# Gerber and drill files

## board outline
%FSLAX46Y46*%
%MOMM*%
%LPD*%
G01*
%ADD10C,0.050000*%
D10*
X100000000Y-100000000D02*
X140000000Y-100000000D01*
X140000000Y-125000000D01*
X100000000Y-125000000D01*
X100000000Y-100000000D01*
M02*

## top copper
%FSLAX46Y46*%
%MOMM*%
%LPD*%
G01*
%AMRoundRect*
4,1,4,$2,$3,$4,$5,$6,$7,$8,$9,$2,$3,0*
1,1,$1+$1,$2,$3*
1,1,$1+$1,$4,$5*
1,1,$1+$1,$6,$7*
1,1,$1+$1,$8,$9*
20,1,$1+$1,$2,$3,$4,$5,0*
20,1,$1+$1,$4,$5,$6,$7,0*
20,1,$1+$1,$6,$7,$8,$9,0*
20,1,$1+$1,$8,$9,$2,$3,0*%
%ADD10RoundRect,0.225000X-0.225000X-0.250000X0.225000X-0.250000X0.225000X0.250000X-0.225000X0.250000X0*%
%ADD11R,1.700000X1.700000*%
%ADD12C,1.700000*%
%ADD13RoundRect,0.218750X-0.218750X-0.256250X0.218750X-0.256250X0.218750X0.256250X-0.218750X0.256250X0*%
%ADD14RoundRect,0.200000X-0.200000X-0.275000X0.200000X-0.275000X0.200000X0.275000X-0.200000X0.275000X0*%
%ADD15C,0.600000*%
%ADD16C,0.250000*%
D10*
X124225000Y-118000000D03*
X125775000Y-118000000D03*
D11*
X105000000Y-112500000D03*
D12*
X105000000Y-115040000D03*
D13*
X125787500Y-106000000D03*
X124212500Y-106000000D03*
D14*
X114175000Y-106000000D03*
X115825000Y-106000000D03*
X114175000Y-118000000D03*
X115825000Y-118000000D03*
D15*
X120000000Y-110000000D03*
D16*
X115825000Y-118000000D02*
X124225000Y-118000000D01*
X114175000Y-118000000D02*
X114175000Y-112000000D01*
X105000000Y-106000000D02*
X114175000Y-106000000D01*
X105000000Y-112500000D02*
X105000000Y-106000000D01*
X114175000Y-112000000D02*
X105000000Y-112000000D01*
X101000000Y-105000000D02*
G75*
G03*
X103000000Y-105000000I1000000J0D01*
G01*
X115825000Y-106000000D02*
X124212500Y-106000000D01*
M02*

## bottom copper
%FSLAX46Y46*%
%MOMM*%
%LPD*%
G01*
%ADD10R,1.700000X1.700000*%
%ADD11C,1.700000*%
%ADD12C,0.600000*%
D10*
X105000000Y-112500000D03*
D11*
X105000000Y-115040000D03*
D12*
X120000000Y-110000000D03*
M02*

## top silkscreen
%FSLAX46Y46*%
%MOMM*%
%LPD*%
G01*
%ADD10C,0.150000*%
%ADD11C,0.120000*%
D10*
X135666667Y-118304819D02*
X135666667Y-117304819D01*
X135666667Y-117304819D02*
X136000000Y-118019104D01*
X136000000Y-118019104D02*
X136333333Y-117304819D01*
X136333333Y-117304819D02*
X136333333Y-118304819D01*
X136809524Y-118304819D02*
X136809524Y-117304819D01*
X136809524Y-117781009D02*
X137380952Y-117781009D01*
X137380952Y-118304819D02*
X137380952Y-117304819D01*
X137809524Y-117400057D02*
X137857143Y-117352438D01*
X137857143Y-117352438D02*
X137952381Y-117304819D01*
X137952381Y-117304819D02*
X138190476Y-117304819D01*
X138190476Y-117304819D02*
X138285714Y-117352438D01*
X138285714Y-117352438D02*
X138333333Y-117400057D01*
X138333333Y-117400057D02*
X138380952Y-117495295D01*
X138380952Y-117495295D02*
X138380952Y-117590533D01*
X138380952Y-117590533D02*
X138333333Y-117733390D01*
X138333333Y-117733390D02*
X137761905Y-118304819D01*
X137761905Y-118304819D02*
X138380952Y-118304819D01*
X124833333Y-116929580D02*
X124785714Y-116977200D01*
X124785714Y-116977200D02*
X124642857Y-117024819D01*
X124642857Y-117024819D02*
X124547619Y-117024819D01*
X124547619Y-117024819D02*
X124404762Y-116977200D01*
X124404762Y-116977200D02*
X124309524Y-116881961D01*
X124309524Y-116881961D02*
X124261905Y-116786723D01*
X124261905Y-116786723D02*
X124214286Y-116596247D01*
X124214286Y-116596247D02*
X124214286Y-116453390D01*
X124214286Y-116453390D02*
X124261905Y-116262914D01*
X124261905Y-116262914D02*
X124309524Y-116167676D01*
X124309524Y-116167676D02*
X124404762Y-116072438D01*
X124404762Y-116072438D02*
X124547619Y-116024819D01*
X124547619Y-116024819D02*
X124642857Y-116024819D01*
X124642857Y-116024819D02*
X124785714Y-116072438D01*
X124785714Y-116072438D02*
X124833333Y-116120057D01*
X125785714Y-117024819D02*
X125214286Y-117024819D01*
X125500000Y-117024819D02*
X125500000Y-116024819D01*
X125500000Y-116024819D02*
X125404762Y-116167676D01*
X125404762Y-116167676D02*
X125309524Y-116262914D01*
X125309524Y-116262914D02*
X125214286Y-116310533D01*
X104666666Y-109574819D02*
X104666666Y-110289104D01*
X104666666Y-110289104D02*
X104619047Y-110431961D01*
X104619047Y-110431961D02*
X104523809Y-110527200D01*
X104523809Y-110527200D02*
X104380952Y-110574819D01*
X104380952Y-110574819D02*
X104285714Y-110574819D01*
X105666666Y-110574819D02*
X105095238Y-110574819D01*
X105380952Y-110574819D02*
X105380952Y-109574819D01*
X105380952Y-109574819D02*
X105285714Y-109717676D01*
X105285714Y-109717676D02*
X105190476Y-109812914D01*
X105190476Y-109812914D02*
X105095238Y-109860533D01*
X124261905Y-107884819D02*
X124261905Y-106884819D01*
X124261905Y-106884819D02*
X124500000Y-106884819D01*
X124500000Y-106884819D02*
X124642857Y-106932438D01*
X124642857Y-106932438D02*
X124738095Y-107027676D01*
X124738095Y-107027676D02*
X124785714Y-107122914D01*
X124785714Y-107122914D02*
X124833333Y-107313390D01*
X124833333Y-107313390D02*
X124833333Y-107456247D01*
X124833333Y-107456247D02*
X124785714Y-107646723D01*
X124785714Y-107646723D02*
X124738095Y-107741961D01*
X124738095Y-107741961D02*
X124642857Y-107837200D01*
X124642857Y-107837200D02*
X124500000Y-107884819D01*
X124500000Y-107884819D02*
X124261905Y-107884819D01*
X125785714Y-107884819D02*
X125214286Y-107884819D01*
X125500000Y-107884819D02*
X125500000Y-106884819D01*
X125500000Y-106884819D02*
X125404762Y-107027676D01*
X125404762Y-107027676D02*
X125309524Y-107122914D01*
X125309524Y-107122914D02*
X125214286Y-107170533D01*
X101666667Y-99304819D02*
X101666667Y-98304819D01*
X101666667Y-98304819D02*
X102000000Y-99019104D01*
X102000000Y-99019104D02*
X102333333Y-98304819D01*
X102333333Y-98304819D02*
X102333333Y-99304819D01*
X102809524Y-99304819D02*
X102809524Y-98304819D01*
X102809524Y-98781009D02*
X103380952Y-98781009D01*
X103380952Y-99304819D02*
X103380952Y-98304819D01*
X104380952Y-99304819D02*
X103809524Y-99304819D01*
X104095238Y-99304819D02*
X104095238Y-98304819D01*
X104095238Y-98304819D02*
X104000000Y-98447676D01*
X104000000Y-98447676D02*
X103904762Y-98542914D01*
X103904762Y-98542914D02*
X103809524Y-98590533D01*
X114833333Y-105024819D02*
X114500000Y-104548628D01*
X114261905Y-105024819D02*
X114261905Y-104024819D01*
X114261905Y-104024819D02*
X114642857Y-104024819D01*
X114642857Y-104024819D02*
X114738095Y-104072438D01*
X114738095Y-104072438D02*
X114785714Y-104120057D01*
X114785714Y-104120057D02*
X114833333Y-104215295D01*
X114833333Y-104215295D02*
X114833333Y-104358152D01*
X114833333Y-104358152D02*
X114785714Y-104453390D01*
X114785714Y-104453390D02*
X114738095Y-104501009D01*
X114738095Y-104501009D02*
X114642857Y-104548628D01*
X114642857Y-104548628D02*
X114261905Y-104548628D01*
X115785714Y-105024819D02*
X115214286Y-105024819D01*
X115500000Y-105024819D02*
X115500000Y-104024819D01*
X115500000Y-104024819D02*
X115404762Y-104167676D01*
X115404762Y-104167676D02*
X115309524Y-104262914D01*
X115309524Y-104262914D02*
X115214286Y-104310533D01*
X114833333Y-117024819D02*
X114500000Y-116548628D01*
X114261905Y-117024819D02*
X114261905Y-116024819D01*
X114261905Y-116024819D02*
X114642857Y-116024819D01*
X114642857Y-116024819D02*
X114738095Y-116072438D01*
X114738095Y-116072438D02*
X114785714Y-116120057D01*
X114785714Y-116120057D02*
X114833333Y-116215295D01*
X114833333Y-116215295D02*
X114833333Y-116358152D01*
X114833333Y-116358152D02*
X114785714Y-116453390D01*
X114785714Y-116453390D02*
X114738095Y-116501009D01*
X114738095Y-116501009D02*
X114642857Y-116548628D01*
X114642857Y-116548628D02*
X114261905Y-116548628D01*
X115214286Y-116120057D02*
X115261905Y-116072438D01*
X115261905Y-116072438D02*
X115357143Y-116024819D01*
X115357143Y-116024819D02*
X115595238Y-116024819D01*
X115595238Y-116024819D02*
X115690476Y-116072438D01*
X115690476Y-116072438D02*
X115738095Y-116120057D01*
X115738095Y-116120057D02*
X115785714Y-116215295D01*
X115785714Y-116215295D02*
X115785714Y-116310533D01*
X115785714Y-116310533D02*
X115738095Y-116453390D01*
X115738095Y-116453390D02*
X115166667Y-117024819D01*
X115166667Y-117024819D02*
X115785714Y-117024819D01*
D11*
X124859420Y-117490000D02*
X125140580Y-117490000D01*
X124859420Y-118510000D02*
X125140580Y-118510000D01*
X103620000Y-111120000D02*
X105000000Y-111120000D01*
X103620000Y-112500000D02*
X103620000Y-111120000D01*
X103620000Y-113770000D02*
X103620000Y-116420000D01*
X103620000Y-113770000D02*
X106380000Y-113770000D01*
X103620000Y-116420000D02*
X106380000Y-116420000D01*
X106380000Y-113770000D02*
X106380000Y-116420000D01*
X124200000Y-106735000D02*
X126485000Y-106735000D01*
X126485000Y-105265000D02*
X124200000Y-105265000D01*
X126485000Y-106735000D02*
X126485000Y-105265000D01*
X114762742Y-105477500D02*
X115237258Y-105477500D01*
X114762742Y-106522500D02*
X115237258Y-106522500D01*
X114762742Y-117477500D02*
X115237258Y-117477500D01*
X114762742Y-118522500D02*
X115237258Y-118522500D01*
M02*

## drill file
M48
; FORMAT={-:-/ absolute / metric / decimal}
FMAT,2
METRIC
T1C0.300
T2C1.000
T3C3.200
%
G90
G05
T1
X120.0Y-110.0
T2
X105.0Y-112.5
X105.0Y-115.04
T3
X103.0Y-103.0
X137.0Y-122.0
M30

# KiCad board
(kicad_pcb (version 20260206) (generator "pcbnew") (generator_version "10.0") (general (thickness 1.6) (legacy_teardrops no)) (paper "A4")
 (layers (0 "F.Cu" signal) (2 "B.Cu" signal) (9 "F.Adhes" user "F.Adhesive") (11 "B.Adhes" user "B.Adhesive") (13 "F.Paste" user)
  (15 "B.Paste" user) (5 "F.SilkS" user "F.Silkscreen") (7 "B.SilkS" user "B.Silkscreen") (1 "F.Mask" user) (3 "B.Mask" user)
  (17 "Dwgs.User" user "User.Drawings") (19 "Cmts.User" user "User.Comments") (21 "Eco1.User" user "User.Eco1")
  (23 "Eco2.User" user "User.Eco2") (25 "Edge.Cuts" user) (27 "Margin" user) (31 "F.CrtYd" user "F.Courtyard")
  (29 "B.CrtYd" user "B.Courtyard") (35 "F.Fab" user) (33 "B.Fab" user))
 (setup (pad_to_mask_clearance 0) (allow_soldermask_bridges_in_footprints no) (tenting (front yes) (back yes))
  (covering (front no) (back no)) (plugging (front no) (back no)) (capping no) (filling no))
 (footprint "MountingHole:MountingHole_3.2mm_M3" (layer "F.Cu") (at 137 122)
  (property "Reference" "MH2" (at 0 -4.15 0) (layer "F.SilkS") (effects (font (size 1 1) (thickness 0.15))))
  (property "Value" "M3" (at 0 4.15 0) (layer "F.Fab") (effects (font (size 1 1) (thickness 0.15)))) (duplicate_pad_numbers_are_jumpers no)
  (pad "" np_thru_hole circle (at 0 0) (size 3.2 3.2) (drill 3.2) (layers "*.Cu" "*.Mask")))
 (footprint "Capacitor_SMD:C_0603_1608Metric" (layer "F.Cu") (at 125 118)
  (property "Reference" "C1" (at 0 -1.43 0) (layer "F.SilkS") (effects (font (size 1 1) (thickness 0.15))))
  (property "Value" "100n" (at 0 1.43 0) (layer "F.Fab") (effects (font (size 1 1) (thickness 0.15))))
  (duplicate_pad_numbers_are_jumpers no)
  (fp_line (start -0.14058 -0.51) (end 0.14058 -0.51) (stroke (width 0.12) (type solid)) (layer "F.SilkS"))
  (fp_line (start -0.14058 0.51) (end 0.14058 0.51) (stroke (width 0.12) (type solid)) (layer "F.SilkS"))
  (pad "1" smd roundrect (at -0.775 0) (size 0.9 0.95) (layers "F.Cu" "F.Mask" "F.Paste") (roundrect_rratio 0.25) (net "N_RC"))
  (pad "2" smd roundrect (at 0.775 0) (size 0.9 0.95) (layers "F.Cu" "F.Mask" "F.Paste") (roundrect_rratio 0.25) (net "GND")))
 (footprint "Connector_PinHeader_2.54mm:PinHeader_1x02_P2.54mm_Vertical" (layer "F.Cu") (at 105 112.5)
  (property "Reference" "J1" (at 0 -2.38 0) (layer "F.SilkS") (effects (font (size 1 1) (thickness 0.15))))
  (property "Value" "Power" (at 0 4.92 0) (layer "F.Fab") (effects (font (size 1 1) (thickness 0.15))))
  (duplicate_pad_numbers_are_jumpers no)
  (fp_line (start -1.38 -1.38) (end 0 -1.38) (stroke (width 0.12) (type solid)) (layer "F.SilkS"))
  (fp_line (start -1.38 0) (end -1.38 -1.38) (stroke (width 0.12) (type solid)) (layer "F.SilkS"))
  (fp_line (start -1.38 1.27) (end -1.38 3.92) (stroke (width 0.12) (type solid)) (layer "F.SilkS"))
  (fp_line (start -1.38 1.27) (end 1.38 1.27) (stroke (width 0.12) (type solid)) (layer "F.SilkS"))
  (fp_line (start -1.38 3.92) (end 1.38 3.92) (stroke (width 0.12) (type solid)) (layer "F.SilkS"))
  (fp_line (start 1.38 1.27) (end 1.38 3.92) (stroke (width 0.12) (type solid)) (layer "F.SilkS"))
  (pad "1" thru_hole rect (at 0 0) (size 1.7 1.7) (drill 1) (layers "*.Cu" "*.Mask") (remove_unused_layers no) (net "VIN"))
  (pad "2" thru_hole circle (at 0 2.54) (size 1.7 1.7) (drill 1) (layers "*.Cu" "*.Mask") (remove_unused_layers no) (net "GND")))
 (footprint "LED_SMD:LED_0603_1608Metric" (layer "F.Cu") (at 125 106 180)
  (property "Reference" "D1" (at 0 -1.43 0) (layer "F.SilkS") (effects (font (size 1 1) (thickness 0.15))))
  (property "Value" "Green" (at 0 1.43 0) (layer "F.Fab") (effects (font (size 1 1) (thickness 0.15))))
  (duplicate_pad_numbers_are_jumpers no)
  (fp_line (start 0.8 -0.735) (end -1.485 -0.735) (stroke (width 0.12) (type solid)) (layer "F.SilkS"))
  (fp_line (start -1.485 0.735) (end 0.8 0.735) (stroke (width 0.12) (type solid)) (layer "F.SilkS"))
  (fp_line (start -1.485 -0.735) (end -1.485 0.735) (stroke (width 0.12) (type solid)) (layer "F.SilkS"))
  (pad "1" smd roundrect (at -0.7875 0) (size 0.875 0.95) (layers "F.Cu" "F.Mask" "F.Paste") (roundrect_rratio 0.25) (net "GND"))
  (pad "2" smd roundrect (at 0.7875 0) (size 0.875 0.95) (layers "F.Cu" "F.Mask" "F.Paste") (roundrect_rratio 0.25) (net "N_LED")))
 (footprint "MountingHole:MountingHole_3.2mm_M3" (layer "F.Cu") (at 103 103)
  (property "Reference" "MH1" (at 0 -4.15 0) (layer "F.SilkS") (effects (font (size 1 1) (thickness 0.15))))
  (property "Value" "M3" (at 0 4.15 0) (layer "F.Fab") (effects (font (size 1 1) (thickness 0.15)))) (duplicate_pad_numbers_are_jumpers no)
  (pad "" np_thru_hole circle (at 0 0) (size 3.2 3.2) (drill 3.2) (layers "*.Cu" "*.Mask")))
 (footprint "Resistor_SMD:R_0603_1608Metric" (layer "F.Cu") (at 115 106)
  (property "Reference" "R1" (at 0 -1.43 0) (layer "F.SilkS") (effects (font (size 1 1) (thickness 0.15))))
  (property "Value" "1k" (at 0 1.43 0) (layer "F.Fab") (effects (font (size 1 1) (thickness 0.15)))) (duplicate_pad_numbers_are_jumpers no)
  (fp_line (start -0.237258 -0.5225) (end 0.237258 -0.5225) (stroke (width 0.12) (type solid)) (layer "F.SilkS"))
  (fp_line (start -0.237258 0.5225) (end 0.237258 0.5225) (stroke (width 0.12) (type solid)) (layer "F.SilkS"))
  (pad "1" smd roundrect (at -0.825 0) (size 0.8 0.95) (layers "F.Cu" "F.Mask" "F.Paste") (roundrect_rratio 0.25) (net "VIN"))
  (pad "2" smd roundrect (at 0.825 0) (size 0.8 0.95) (layers "F.Cu" "F.Mask" "F.Paste") (roundrect_rratio 0.25) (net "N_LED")))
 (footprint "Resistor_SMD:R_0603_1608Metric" (layer "F.Cu") (at 115 118)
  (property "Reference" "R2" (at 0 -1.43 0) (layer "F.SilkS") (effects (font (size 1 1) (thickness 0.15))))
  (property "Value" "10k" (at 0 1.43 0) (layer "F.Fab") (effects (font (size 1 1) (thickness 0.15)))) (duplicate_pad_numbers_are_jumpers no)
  (fp_line (start -0.237258 -0.5225) (end 0.237258 -0.5225) (stroke (width 0.12) (type solid)) (layer "F.SilkS"))
  (fp_line (start -0.237258 0.5225) (end 0.237258 0.5225) (stroke (width 0.12) (type solid)) (layer "F.SilkS"))
  (pad "1" smd roundrect (at -0.825 0) (size 0.8 0.95) (layers "F.Cu" "F.Mask" "F.Paste") (roundrect_rratio 0.25) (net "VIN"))
  (pad "2" smd roundrect (at 0.825 0) (size 0.8 0.95) (layers "F.Cu" "F.Mask" "F.Paste") (roundrect_rratio 0.25) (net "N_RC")))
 (gr_rect (start 100 100) (end 140 125) (stroke (width 0.05) (type default)) (fill no) (layer "Edge.Cuts"))
 (segment (start 115.825 118) (end 124.225 118) (width 0.25) (layer "F.Cu") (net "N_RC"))
 (segment (start 114.175 118) (end 114.175 112) (width 0.25) (layer "F.Cu") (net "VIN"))
 (segment (start 105 106) (end 114.175 106) (width 0.25) (layer "F.Cu") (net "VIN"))
 (segment (start 105 112.5) (end 105 106) (width 0.25) (layer "F.Cu") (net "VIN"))
 (segment (start 114.175 112) (end 105 112) (width 0.25) (layer "F.Cu") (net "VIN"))
 (via (at 120 110) (size 0.6) (drill 0.3) (layers "F.Cu" "B.Cu") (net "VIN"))
 (arc (start 101 105) (mid 102 106) (end 103 105) (width 0.25) (layer "F.Cu") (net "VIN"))
 (segment (start 115.825 106) (end 124.2125 106) (width 0.25) (layer "F.Cu") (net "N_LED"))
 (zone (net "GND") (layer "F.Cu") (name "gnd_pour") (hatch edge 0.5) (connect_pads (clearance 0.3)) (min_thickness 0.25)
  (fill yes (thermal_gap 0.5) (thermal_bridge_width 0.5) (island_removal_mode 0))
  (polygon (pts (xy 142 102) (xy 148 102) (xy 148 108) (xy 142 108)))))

